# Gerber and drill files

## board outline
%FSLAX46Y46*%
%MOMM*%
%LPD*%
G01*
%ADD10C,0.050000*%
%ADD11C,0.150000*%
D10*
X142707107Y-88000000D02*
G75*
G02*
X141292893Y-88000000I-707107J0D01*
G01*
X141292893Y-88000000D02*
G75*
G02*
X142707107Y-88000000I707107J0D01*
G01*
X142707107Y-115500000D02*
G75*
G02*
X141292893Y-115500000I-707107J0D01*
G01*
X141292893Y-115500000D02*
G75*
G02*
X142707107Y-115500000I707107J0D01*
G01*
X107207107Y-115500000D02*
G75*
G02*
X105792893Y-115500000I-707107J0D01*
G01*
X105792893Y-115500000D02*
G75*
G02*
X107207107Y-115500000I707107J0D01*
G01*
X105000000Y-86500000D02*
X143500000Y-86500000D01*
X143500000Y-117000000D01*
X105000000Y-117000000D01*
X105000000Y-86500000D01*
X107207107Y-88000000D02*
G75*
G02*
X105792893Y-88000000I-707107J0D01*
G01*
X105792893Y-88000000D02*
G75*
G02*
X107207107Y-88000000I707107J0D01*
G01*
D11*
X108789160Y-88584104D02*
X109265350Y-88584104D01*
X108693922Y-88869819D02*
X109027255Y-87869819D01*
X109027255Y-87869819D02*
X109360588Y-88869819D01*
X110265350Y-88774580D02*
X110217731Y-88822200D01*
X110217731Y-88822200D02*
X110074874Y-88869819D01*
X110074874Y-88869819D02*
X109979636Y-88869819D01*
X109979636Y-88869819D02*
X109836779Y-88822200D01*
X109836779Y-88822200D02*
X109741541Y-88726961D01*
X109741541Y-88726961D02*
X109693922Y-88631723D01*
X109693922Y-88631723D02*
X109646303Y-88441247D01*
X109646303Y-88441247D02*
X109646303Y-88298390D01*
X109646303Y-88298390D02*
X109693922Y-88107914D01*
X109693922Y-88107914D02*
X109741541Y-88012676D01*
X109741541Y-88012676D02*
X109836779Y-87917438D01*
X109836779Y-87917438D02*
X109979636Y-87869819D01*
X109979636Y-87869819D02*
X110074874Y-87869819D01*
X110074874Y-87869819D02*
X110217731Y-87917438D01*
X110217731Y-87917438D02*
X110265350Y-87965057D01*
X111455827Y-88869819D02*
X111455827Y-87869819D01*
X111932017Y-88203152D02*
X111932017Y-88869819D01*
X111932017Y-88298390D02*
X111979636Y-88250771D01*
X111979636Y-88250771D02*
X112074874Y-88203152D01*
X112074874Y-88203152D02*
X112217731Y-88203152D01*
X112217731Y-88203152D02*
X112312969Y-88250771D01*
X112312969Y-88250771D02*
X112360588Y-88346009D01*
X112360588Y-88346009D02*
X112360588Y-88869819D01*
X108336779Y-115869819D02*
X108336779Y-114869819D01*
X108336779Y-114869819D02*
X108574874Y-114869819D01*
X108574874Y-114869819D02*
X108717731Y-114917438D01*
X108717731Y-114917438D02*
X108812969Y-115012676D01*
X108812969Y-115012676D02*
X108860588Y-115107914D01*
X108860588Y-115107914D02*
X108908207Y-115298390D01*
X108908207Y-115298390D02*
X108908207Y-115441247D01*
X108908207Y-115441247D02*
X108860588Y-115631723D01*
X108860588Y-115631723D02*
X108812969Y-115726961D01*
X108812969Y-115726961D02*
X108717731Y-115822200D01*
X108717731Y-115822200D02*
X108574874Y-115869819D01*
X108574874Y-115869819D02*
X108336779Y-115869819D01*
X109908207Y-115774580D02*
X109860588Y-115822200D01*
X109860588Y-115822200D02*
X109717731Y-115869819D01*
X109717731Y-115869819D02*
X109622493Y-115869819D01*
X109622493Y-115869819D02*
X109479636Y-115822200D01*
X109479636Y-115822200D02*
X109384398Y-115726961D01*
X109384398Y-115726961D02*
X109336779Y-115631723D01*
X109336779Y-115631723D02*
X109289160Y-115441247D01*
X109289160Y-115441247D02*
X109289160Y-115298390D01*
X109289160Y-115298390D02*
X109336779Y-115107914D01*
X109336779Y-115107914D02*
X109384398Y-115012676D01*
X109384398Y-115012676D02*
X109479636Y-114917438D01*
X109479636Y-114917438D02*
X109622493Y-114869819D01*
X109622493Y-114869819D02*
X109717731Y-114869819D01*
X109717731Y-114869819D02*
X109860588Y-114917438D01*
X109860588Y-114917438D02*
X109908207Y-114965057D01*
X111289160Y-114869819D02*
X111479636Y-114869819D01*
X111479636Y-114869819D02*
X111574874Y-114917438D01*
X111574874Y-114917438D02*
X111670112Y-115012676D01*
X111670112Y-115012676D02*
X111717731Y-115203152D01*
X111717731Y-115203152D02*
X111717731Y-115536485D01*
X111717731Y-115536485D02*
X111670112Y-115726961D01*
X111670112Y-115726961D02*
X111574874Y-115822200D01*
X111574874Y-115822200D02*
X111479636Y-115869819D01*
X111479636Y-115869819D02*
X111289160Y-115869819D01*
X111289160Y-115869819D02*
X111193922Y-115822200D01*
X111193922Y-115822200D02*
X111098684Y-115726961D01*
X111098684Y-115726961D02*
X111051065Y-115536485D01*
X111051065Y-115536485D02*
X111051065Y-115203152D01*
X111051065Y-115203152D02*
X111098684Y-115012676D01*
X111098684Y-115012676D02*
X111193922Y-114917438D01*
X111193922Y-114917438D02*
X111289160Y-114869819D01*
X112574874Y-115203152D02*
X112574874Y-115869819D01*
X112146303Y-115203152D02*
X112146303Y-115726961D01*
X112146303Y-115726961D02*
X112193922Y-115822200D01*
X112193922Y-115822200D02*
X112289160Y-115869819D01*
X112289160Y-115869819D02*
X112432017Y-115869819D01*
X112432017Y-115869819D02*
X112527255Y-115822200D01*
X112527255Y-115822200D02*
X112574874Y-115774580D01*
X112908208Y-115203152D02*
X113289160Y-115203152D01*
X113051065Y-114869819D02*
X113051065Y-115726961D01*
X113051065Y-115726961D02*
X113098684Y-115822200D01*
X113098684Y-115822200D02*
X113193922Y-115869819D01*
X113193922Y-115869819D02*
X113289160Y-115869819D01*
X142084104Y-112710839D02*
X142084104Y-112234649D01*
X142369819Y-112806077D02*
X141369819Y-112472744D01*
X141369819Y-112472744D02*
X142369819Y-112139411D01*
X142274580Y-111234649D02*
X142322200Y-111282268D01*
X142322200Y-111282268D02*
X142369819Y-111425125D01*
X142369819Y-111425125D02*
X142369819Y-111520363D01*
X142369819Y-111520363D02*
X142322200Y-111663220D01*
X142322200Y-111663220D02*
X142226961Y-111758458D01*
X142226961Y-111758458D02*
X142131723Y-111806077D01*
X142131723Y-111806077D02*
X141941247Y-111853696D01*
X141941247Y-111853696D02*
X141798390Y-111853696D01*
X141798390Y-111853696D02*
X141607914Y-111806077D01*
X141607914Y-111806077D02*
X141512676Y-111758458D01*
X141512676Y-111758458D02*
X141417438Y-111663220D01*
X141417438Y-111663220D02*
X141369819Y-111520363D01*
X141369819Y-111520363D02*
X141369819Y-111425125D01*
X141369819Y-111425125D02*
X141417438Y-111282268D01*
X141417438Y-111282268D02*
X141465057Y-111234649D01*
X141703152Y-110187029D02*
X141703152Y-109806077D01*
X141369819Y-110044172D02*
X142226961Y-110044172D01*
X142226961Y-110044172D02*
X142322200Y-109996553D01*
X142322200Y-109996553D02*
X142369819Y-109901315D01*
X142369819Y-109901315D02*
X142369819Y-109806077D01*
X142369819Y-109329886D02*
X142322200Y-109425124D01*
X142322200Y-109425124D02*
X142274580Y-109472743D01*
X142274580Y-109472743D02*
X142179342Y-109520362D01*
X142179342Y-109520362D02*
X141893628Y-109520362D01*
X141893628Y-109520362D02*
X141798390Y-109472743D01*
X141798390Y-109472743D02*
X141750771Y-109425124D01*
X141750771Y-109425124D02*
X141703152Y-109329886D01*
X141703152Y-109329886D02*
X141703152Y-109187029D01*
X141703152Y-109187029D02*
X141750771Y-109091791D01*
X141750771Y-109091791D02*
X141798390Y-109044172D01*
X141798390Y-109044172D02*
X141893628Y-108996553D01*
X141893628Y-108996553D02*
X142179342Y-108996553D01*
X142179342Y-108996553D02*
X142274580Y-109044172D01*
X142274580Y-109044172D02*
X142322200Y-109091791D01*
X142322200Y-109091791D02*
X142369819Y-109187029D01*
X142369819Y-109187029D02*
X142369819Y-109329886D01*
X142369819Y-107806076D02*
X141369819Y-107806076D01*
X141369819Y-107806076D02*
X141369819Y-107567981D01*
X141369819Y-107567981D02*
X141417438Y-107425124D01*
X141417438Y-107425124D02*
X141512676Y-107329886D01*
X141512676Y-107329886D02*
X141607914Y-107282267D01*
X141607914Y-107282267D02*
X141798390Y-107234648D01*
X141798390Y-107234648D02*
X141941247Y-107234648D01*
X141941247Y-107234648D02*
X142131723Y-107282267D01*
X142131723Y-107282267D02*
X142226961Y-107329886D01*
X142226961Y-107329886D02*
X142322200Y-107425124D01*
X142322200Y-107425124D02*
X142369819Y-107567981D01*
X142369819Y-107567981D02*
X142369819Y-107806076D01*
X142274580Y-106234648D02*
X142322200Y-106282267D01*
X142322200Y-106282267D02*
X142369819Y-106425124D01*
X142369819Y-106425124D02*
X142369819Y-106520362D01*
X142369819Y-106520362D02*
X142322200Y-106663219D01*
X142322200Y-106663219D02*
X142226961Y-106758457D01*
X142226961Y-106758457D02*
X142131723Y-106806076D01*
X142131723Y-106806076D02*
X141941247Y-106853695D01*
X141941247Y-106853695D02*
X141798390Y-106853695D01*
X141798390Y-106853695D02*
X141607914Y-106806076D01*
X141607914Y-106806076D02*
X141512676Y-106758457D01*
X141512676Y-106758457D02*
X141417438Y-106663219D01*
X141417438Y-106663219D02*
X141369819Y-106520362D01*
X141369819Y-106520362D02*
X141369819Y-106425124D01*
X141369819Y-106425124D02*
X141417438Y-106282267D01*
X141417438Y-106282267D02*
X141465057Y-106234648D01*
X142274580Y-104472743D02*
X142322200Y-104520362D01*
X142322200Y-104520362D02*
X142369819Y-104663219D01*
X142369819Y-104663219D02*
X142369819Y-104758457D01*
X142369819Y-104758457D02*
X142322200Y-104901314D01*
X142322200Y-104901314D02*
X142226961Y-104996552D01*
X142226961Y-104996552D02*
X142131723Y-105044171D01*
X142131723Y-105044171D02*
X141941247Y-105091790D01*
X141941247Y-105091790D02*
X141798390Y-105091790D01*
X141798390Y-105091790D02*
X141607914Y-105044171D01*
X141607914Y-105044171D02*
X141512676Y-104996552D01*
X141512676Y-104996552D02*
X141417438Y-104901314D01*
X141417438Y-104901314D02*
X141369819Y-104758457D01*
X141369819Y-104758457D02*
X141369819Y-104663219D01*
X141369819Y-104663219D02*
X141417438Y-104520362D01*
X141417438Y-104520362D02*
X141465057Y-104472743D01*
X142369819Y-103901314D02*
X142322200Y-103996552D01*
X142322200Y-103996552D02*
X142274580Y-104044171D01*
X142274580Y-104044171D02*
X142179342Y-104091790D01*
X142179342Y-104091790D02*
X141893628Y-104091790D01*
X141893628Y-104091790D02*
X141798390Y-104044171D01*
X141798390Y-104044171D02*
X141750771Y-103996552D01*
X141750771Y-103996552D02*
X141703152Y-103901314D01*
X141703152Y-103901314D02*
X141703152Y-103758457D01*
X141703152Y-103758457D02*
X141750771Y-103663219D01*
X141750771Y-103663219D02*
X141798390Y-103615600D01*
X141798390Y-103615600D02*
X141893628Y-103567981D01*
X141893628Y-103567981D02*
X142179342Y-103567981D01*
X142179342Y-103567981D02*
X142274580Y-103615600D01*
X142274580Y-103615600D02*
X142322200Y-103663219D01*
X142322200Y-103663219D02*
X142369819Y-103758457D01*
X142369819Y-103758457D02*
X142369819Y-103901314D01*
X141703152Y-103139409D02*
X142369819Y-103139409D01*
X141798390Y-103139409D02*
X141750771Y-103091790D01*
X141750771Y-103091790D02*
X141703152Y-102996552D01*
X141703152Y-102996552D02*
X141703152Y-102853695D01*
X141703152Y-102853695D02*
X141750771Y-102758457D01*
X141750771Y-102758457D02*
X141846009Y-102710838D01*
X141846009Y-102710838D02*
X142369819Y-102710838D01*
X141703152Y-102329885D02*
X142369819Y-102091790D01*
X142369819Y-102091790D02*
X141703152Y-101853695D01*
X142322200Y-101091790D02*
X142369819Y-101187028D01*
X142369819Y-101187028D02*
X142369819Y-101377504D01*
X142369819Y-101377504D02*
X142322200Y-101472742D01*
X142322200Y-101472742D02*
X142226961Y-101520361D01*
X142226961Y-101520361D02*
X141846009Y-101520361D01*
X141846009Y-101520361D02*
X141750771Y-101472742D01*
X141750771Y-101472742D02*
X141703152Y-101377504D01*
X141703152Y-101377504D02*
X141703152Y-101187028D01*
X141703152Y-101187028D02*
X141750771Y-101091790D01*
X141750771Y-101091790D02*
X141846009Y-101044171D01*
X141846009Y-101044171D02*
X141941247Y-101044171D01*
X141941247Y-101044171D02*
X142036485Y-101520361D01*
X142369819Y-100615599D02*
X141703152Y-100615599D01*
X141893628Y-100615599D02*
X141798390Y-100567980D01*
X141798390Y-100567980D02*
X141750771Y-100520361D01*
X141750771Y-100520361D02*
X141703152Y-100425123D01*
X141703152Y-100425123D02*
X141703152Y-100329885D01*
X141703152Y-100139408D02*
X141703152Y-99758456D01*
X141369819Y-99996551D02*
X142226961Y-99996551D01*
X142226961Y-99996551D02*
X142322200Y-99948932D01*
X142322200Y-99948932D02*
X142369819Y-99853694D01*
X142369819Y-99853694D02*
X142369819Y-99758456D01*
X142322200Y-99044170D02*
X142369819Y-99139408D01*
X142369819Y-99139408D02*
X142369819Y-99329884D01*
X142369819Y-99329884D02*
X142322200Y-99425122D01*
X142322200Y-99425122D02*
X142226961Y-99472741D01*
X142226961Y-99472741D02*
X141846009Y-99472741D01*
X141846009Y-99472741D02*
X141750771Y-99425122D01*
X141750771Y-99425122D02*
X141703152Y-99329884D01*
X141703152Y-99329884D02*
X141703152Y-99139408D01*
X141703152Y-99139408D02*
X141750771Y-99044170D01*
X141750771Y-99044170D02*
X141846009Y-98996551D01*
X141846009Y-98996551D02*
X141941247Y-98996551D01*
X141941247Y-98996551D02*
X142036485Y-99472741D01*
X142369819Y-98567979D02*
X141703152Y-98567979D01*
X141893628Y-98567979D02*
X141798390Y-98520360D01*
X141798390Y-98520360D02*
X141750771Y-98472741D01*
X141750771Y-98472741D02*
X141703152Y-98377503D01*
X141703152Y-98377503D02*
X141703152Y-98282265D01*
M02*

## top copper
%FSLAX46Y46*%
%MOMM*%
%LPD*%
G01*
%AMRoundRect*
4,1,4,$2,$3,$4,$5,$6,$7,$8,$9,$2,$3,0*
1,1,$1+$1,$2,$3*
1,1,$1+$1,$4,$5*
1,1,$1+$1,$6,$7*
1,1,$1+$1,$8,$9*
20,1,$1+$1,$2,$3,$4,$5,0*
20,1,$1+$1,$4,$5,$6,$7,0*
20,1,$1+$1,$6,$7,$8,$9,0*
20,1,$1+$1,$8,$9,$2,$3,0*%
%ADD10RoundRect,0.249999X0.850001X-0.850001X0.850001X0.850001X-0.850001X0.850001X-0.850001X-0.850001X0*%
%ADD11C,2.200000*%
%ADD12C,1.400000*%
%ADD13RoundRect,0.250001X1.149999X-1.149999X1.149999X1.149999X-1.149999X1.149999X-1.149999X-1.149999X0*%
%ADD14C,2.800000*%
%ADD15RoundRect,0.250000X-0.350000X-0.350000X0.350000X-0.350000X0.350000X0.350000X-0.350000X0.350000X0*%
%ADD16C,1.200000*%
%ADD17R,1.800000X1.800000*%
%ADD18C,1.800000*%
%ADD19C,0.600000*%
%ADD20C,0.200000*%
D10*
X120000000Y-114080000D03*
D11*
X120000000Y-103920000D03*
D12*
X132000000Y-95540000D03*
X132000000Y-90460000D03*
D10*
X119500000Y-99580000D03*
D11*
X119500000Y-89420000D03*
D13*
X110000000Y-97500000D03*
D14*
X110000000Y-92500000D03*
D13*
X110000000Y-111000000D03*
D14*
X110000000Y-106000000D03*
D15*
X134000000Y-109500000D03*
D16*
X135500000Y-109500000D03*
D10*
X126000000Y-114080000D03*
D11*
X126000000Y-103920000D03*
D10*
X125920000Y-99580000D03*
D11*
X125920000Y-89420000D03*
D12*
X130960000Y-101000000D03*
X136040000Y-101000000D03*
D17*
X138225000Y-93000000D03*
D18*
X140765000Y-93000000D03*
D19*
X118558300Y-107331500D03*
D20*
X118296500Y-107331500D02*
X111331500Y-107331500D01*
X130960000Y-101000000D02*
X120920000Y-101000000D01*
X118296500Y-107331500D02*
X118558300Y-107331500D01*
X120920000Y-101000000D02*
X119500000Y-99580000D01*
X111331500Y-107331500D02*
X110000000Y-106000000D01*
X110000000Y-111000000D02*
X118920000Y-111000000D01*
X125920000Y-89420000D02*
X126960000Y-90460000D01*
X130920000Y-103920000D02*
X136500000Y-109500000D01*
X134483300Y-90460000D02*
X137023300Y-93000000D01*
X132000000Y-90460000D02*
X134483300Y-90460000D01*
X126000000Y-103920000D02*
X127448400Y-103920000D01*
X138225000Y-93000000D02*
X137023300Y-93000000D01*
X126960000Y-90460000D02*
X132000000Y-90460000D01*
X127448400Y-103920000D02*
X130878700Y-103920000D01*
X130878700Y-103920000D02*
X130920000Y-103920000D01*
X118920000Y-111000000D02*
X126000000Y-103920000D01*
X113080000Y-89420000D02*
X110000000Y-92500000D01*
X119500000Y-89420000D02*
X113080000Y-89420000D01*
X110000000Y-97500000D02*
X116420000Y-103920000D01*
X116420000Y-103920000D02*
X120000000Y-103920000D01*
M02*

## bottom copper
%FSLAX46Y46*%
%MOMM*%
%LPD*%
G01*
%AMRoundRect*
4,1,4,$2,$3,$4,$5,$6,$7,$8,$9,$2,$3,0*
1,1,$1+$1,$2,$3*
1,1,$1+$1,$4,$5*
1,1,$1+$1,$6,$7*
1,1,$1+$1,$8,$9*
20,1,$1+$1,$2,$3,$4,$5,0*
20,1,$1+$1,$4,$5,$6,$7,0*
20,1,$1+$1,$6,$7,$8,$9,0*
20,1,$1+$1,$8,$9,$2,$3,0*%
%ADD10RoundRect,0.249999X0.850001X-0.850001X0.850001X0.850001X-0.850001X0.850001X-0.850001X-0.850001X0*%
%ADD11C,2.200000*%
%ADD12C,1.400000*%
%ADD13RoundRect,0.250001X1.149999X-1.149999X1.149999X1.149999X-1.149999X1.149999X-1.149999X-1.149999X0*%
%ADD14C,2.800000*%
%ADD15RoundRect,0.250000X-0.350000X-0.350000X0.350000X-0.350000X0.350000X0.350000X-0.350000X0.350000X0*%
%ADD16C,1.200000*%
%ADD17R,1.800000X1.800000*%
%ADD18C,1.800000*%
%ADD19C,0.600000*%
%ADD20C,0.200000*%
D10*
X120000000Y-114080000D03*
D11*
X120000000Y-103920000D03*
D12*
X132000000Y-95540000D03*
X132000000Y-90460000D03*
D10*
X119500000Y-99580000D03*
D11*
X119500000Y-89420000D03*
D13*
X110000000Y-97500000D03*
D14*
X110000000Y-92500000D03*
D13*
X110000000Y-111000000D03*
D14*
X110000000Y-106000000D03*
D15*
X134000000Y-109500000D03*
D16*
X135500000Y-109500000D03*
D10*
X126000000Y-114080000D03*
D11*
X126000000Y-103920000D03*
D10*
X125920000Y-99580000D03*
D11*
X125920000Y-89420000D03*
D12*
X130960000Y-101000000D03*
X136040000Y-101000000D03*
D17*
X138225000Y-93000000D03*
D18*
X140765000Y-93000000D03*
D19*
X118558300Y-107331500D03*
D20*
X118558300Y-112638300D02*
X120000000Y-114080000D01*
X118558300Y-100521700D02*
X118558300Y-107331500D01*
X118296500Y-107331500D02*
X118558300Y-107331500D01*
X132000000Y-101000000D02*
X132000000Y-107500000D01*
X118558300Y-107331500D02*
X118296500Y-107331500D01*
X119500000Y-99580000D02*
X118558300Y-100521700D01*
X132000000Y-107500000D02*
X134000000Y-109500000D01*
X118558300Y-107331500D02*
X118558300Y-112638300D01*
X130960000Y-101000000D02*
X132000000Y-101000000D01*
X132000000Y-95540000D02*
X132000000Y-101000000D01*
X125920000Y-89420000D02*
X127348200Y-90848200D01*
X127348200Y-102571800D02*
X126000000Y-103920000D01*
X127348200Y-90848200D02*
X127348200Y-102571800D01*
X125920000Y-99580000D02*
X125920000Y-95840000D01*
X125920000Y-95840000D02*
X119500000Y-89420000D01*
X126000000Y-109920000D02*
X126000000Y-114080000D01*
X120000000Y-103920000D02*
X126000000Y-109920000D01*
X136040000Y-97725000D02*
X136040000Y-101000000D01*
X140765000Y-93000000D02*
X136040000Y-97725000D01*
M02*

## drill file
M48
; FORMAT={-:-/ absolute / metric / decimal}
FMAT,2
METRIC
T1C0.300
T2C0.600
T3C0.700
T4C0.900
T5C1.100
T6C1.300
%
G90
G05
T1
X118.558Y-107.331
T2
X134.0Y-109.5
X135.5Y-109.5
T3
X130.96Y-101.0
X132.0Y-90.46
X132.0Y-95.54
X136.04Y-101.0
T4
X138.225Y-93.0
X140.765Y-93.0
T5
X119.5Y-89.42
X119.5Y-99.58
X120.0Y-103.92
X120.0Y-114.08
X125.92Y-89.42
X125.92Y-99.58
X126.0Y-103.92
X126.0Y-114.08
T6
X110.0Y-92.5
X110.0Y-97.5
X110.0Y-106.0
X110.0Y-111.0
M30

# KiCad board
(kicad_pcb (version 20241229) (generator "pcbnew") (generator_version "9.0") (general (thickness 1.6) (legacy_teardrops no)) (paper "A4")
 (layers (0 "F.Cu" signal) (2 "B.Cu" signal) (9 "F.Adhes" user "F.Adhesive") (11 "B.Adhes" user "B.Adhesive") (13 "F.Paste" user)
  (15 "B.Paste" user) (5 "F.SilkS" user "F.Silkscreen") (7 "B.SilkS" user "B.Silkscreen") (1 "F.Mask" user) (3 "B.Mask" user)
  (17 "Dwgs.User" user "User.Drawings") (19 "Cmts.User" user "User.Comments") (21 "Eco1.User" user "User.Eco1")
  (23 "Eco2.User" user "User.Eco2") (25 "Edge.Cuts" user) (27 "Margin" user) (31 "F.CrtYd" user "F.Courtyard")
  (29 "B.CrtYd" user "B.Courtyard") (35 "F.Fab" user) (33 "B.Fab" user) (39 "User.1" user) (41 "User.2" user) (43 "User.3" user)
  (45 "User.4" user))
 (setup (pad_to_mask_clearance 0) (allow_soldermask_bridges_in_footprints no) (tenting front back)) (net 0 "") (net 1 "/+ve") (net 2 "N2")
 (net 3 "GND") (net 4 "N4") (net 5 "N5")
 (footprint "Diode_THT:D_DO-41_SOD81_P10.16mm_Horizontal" (layer "F.Cu") (at 120 114.08 90)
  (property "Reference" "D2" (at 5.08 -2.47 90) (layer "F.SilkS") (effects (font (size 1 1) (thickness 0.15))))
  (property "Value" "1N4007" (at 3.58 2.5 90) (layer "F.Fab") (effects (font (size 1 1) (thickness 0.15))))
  (pad "1" thru_hole roundrect (at 0 0 90) (size 2.2 2.2) (drill 1.1) (layers "*.Cu" "*.Mask") (remove_unused_layers no)
   (roundrect_rratio 0.113636) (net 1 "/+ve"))
  (pad "2" thru_hole circle (at 10.16 0 90) (size 2.2 2.2) (drill 1.1) (layers "*.Cu" "*.Mask") (remove_unused_layers no) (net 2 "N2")))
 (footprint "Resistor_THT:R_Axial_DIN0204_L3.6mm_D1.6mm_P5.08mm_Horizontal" (layer "F.Cu") (at 132 95.54 90)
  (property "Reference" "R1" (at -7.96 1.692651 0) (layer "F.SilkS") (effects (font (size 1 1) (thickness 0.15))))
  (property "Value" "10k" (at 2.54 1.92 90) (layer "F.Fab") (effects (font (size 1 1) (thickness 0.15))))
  (pad "1" thru_hole circle (at 0 0 90) (size 1.4 1.4) (drill 0.7) (layers "*.Cu" "*.Mask") (remove_unused_layers no) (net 1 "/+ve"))
  (pad "2" thru_hole circle (at 5.08 0 90) (size 1.4 1.4) (drill 0.7) (layers "*.Cu" "*.Mask") (remove_unused_layers no) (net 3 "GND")))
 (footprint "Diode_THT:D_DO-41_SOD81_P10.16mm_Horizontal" (layer "F.Cu") (at 119.5 99.58 90)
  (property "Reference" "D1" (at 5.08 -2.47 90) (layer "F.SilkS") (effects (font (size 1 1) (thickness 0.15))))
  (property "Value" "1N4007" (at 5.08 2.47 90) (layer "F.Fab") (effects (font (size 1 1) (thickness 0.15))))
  (pad "1" thru_hole roundrect (at 0 0 90) (size 2.2 2.2) (drill 1.1) (layers "*.Cu" "*.Mask") (remove_unused_layers no)
   (roundrect_rratio 0.113636) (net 1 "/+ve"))
  (pad "2" thru_hole circle (at 10.16 0 90) (size 2.2 2.2) (drill 1.1) (layers "*.Cu" "*.Mask") (remove_unused_layers no) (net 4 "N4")))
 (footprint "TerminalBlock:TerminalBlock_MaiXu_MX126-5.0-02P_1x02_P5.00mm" (layer "F.Cu") (at 110 97.5 90)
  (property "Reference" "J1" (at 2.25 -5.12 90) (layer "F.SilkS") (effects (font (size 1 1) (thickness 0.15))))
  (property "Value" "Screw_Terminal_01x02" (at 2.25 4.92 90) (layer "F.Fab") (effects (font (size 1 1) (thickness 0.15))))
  (pad "1" thru_hole roundrect (at 0 0 90) (size 2.8 2.8) (drill 1.3) (layers "*.Cu" "*.Mask") (remove_unused_layers no)
   (roundrect_rratio 0.089286) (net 2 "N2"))
  (pad "2" thru_hole circle (at 5 0 90) (size 2.8 2.8) (drill 1.3) (layers "*.Cu" "*.Mask") (remove_unused_layers no) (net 4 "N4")))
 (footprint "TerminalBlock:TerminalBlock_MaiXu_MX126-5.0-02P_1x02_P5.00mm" (layer "F.Cu") (at 110 111 90)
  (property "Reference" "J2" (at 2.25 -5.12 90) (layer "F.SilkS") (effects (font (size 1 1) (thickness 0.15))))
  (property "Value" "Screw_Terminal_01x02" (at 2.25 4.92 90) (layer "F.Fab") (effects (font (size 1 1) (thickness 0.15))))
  (pad "1" thru_hole roundrect (at 0 0 90) (size 2.8 2.8) (drill 1.3) (layers "*.Cu" "*.Mask") (remove_unused_layers no)
   (roundrect_rratio 0.089286) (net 3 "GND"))
  (pad "2" thru_hole circle (at 5 0 90) (size 2.8 2.8) (drill 1.3) (layers "*.Cu" "*.Mask") (remove_unused_layers no) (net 1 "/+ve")))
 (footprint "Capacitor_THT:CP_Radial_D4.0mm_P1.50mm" (layer "F.Cu") (at 134 109.5)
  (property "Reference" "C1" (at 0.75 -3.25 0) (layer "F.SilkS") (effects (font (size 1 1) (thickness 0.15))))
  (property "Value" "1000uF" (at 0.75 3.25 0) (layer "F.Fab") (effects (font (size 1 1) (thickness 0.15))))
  (pad "1" thru_hole roundrect (at 0 0) (size 1.2 1.2) (drill 0.6) (layers "*.Cu" "*.Mask") (remove_unused_layers no)
   (roundrect_rratio 0.208333) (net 1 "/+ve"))
  (pad "2" thru_hole circle (at 1.5 0) (size 1.2 1.2) (drill 0.6) (layers "*.Cu" "*.Mask") (remove_unused_layers no) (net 3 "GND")))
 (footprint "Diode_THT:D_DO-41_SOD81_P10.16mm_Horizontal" (layer "F.Cu") (at 126 114.08 90)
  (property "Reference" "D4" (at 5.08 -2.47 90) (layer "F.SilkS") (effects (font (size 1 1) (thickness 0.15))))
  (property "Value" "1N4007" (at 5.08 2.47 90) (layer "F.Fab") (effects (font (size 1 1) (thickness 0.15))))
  (pad "1" thru_hole roundrect (at 0 0 90) (size 2.2 2.2) (drill 1.1) (layers "*.Cu" "*.Mask") (remove_unused_layers no)
   (roundrect_rratio 0.113636) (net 2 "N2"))
  (pad "2" thru_hole circle (at 10.16 0 90) (size 2.2 2.2) (drill 1.1) (layers "*.Cu" "*.Mask") (remove_unused_layers no) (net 3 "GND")))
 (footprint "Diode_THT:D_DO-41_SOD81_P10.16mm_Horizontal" (layer "F.Cu") (at 125.92 99.58 90)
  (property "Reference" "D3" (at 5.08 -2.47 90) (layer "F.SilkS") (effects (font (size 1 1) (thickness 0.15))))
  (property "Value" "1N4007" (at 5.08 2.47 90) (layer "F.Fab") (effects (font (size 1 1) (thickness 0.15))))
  (pad "1" thru_hole roundrect (at 0 0 90) (size 2.2 2.2) (drill 1.1) (layers "*.Cu" "*.Mask") (remove_unused_layers no)
   (roundrect_rratio 0.113636) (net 4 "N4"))
  (pad "2" thru_hole circle (at 10.16 0 90) (size 2.2 2.2) (drill 1.1) (layers "*.Cu" "*.Mask") (remove_unused_layers no) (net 3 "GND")))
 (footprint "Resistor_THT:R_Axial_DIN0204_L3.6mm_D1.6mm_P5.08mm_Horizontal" (layer "F.Cu") (at 130.96 101)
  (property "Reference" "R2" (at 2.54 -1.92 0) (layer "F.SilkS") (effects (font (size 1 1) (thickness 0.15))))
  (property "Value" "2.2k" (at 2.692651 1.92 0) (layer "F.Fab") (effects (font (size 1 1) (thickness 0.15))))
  (pad "1" thru_hole circle (at 0 0) (size 1.4 1.4) (drill 0.7) (layers "*.Cu" "*.Mask") (remove_unused_layers no) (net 1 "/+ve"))
  (pad "2" thru_hole circle (at 5.08 0) (size 1.4 1.4) (drill 0.7) (layers "*.Cu" "*.Mask") (remove_unused_layers no) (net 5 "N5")))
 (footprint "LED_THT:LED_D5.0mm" (layer "F.Cu") (at 138.225 93)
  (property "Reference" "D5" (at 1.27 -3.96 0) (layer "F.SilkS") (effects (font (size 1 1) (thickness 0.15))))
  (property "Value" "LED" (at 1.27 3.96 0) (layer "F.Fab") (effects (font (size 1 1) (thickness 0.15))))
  (pad "1" thru_hole rect (at 0 0) (size 1.8 1.8) (drill 0.9) (layers "*.Cu" "*.Mask") (remove_unused_layers no) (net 3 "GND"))
  (pad "2" thru_hole circle (at 2.54 0) (size 1.8 1.8) (drill 0.9) (layers "*.Cu" "*.Mask") (remove_unused_layers no) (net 5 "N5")))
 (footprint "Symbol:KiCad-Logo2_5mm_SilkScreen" (layer "B.Cu") (at 121.5 109 180)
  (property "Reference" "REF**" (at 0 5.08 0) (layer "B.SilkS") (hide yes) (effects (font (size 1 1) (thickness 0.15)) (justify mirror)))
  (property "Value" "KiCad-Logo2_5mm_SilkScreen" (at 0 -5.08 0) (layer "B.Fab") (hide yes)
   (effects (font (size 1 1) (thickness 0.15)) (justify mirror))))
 (gr_circle (center 142 88) (end 142.5 87.5) (stroke (width 0.05) (type default)) (fill no) (layer "Edge.Cuts"))
 (gr_circle (center 142 115.5) (end 142.5 115) (stroke (width 0.05) (type default)) (fill no) (layer "Edge.Cuts"))
 (gr_circle (center 106.5 115.5) (end 107 115) (stroke (width 0.05) (type default)) (fill no) (layer "Edge.Cuts"))
 (gr_rect (start 105 86.5) (end 143.5 117) (stroke (width 0.05) (type default)) (fill no) (layer "Edge.Cuts"))
 (gr_circle (center 106.5 88) (end 107 87.5) (stroke (width 0.05) (type default)) (fill no) (layer "Edge.Cuts"))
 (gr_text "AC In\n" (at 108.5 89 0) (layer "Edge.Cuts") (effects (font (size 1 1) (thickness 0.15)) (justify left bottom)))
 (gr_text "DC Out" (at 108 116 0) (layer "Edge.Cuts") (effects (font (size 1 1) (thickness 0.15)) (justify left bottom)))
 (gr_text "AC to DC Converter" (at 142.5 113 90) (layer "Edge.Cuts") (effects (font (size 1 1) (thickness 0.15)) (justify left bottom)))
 (segment (start 118.2965 107.3315) (end 111.3315 107.3315) (width 0.2) (layer "F.Cu") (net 1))
 (segment (start 130.96 101) (end 120.92 101) (width 0.2) (layer "F.Cu") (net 1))
 (segment (start 118.2965 107.3315) (end 118.5583 107.3315) (width 0.2) (layer "F.Cu") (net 1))
 (segment (start 120.92 101) (end 119.5 99.58) (width 0.2) (layer "F.Cu") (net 1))
 (segment (start 111.3315 107.3315) (end 110 106) (width 0.2) (layer "F.Cu") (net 1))
 (via (at 118.5583 107.3315) (size 0.6) (drill 0.3) (layers "F.Cu" "B.Cu") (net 1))
 (segment (start 118.5583 112.6383) (end 120 114.08) (width 0.2) (layer "B.Cu") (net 1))
 (segment (start 118.5583 100.5217) (end 118.5583 107.3315) (width 0.2) (layer "B.Cu") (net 1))
 (segment (start 118.2965 107.3315) (end 118.5583 107.3315) (width 0.2) (layer "B.Cu") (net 1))
 (segment (start 132 101) (end 132 107.5) (width 0.2) (layer "B.Cu") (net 1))
 (segment (start 118.5583 107.3315) (end 118.2965 107.3315) (width 0.2) (layer "B.Cu") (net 1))
 (segment (start 119.5 99.58) (end 118.5583 100.5217) (width 0.2) (layer "B.Cu") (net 1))
 (segment (start 132 107.5) (end 134 109.5) (width 0.2) (layer "B.Cu") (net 1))
 (segment (start 118.5583 107.3315) (end 118.5583 112.6383) (width 0.2) (layer "B.Cu") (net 1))
 (segment (start 130.96 101) (end 132 101) (width 0.2) (layer "B.Cu") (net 1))
 (segment (start 132 95.54) (end 132 101) (width 0.2) (layer "B.Cu") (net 1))
 (segment (start 110 111) (end 118.92 111) (width 0.2) (layer "F.Cu") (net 3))
 (segment (start 125.92 89.42) (end 126.96 90.46) (width 0.2) (layer "F.Cu") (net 3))
 (segment (start 130.92 103.92) (end 136.5 109.5) (width 0.2) (layer "F.Cu") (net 3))
 (segment (start 134.4833 90.46) (end 137.0233 93) (width 0.2) (layer "F.Cu") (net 3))
 (segment (start 132 90.46) (end 134.4833 90.46) (width 0.2) (layer "F.Cu") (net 3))
 (segment (start 126 103.92) (end 127.4484 103.92) (width 0.2) (layer "F.Cu") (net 3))
 (segment (start 138.225 93) (end 137.0233 93) (width 0.2) (layer "F.Cu") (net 3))
 (segment (start 126.96 90.46) (end 132 90.46) (width 0.2) (layer "F.Cu") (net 3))
 (segment (start 127.4484 103.92) (end 130.8787 103.92) (width 0.2) (layer "F.Cu") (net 3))
 (segment (start 130.8787 103.92) (end 130.92 103.92) (width 0.2) (layer "F.Cu") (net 3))
 (segment (start 118.92 111) (end 126 103.92) (width 0.2) (layer "F.Cu") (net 3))
 (segment (start 125.92 89.42) (end 127.3482 90.8482) (width 0.2) (layer "B.Cu") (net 3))
 (segment (start 127.3482 102.5718) (end 126 103.92) (width 0.2) (layer "B.Cu") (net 3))
 (segment (start 127.3482 90.8482) (end 127.3482 102.5718) (width 0.2) (layer "B.Cu") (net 3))
 (segment (start 113.08 89.42) (end 110 92.5) (width 0.2) (layer "F.Cu") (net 4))
 (segment (start 119.5 89.42) (end 113.08 89.42) (width 0.2) (layer "F.Cu") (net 4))
 (segment (start 125.92 99.58) (end 125.92 95.84) (width 0.2) (layer "B.Cu") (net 4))
 (segment (start 125.92 95.84) (end 119.5 89.42) (width 0.2) (layer "B.Cu") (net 4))
 (segment (start 110 97.5) (end 116.42 103.92) (width 0.2) (layer "F.Cu") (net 2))
 (segment (start 116.42 103.92) (end 120 103.92) (width 0.2) (layer "F.Cu") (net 2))
 (segment (start 126 109.92) (end 126 114.08) (width 0.2) (layer "B.Cu") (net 2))
 (segment (start 120 103.92) (end 126 109.92) (width 0.2) (layer "B.Cu") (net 2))
 (segment (start 136.04 97.725) (end 136.04 101) (width 0.2) (layer "B.Cu") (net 5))
 (segment (start 140.765 93) (end 136.04 97.725) (width 0.2) (layer "B.Cu") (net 5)))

